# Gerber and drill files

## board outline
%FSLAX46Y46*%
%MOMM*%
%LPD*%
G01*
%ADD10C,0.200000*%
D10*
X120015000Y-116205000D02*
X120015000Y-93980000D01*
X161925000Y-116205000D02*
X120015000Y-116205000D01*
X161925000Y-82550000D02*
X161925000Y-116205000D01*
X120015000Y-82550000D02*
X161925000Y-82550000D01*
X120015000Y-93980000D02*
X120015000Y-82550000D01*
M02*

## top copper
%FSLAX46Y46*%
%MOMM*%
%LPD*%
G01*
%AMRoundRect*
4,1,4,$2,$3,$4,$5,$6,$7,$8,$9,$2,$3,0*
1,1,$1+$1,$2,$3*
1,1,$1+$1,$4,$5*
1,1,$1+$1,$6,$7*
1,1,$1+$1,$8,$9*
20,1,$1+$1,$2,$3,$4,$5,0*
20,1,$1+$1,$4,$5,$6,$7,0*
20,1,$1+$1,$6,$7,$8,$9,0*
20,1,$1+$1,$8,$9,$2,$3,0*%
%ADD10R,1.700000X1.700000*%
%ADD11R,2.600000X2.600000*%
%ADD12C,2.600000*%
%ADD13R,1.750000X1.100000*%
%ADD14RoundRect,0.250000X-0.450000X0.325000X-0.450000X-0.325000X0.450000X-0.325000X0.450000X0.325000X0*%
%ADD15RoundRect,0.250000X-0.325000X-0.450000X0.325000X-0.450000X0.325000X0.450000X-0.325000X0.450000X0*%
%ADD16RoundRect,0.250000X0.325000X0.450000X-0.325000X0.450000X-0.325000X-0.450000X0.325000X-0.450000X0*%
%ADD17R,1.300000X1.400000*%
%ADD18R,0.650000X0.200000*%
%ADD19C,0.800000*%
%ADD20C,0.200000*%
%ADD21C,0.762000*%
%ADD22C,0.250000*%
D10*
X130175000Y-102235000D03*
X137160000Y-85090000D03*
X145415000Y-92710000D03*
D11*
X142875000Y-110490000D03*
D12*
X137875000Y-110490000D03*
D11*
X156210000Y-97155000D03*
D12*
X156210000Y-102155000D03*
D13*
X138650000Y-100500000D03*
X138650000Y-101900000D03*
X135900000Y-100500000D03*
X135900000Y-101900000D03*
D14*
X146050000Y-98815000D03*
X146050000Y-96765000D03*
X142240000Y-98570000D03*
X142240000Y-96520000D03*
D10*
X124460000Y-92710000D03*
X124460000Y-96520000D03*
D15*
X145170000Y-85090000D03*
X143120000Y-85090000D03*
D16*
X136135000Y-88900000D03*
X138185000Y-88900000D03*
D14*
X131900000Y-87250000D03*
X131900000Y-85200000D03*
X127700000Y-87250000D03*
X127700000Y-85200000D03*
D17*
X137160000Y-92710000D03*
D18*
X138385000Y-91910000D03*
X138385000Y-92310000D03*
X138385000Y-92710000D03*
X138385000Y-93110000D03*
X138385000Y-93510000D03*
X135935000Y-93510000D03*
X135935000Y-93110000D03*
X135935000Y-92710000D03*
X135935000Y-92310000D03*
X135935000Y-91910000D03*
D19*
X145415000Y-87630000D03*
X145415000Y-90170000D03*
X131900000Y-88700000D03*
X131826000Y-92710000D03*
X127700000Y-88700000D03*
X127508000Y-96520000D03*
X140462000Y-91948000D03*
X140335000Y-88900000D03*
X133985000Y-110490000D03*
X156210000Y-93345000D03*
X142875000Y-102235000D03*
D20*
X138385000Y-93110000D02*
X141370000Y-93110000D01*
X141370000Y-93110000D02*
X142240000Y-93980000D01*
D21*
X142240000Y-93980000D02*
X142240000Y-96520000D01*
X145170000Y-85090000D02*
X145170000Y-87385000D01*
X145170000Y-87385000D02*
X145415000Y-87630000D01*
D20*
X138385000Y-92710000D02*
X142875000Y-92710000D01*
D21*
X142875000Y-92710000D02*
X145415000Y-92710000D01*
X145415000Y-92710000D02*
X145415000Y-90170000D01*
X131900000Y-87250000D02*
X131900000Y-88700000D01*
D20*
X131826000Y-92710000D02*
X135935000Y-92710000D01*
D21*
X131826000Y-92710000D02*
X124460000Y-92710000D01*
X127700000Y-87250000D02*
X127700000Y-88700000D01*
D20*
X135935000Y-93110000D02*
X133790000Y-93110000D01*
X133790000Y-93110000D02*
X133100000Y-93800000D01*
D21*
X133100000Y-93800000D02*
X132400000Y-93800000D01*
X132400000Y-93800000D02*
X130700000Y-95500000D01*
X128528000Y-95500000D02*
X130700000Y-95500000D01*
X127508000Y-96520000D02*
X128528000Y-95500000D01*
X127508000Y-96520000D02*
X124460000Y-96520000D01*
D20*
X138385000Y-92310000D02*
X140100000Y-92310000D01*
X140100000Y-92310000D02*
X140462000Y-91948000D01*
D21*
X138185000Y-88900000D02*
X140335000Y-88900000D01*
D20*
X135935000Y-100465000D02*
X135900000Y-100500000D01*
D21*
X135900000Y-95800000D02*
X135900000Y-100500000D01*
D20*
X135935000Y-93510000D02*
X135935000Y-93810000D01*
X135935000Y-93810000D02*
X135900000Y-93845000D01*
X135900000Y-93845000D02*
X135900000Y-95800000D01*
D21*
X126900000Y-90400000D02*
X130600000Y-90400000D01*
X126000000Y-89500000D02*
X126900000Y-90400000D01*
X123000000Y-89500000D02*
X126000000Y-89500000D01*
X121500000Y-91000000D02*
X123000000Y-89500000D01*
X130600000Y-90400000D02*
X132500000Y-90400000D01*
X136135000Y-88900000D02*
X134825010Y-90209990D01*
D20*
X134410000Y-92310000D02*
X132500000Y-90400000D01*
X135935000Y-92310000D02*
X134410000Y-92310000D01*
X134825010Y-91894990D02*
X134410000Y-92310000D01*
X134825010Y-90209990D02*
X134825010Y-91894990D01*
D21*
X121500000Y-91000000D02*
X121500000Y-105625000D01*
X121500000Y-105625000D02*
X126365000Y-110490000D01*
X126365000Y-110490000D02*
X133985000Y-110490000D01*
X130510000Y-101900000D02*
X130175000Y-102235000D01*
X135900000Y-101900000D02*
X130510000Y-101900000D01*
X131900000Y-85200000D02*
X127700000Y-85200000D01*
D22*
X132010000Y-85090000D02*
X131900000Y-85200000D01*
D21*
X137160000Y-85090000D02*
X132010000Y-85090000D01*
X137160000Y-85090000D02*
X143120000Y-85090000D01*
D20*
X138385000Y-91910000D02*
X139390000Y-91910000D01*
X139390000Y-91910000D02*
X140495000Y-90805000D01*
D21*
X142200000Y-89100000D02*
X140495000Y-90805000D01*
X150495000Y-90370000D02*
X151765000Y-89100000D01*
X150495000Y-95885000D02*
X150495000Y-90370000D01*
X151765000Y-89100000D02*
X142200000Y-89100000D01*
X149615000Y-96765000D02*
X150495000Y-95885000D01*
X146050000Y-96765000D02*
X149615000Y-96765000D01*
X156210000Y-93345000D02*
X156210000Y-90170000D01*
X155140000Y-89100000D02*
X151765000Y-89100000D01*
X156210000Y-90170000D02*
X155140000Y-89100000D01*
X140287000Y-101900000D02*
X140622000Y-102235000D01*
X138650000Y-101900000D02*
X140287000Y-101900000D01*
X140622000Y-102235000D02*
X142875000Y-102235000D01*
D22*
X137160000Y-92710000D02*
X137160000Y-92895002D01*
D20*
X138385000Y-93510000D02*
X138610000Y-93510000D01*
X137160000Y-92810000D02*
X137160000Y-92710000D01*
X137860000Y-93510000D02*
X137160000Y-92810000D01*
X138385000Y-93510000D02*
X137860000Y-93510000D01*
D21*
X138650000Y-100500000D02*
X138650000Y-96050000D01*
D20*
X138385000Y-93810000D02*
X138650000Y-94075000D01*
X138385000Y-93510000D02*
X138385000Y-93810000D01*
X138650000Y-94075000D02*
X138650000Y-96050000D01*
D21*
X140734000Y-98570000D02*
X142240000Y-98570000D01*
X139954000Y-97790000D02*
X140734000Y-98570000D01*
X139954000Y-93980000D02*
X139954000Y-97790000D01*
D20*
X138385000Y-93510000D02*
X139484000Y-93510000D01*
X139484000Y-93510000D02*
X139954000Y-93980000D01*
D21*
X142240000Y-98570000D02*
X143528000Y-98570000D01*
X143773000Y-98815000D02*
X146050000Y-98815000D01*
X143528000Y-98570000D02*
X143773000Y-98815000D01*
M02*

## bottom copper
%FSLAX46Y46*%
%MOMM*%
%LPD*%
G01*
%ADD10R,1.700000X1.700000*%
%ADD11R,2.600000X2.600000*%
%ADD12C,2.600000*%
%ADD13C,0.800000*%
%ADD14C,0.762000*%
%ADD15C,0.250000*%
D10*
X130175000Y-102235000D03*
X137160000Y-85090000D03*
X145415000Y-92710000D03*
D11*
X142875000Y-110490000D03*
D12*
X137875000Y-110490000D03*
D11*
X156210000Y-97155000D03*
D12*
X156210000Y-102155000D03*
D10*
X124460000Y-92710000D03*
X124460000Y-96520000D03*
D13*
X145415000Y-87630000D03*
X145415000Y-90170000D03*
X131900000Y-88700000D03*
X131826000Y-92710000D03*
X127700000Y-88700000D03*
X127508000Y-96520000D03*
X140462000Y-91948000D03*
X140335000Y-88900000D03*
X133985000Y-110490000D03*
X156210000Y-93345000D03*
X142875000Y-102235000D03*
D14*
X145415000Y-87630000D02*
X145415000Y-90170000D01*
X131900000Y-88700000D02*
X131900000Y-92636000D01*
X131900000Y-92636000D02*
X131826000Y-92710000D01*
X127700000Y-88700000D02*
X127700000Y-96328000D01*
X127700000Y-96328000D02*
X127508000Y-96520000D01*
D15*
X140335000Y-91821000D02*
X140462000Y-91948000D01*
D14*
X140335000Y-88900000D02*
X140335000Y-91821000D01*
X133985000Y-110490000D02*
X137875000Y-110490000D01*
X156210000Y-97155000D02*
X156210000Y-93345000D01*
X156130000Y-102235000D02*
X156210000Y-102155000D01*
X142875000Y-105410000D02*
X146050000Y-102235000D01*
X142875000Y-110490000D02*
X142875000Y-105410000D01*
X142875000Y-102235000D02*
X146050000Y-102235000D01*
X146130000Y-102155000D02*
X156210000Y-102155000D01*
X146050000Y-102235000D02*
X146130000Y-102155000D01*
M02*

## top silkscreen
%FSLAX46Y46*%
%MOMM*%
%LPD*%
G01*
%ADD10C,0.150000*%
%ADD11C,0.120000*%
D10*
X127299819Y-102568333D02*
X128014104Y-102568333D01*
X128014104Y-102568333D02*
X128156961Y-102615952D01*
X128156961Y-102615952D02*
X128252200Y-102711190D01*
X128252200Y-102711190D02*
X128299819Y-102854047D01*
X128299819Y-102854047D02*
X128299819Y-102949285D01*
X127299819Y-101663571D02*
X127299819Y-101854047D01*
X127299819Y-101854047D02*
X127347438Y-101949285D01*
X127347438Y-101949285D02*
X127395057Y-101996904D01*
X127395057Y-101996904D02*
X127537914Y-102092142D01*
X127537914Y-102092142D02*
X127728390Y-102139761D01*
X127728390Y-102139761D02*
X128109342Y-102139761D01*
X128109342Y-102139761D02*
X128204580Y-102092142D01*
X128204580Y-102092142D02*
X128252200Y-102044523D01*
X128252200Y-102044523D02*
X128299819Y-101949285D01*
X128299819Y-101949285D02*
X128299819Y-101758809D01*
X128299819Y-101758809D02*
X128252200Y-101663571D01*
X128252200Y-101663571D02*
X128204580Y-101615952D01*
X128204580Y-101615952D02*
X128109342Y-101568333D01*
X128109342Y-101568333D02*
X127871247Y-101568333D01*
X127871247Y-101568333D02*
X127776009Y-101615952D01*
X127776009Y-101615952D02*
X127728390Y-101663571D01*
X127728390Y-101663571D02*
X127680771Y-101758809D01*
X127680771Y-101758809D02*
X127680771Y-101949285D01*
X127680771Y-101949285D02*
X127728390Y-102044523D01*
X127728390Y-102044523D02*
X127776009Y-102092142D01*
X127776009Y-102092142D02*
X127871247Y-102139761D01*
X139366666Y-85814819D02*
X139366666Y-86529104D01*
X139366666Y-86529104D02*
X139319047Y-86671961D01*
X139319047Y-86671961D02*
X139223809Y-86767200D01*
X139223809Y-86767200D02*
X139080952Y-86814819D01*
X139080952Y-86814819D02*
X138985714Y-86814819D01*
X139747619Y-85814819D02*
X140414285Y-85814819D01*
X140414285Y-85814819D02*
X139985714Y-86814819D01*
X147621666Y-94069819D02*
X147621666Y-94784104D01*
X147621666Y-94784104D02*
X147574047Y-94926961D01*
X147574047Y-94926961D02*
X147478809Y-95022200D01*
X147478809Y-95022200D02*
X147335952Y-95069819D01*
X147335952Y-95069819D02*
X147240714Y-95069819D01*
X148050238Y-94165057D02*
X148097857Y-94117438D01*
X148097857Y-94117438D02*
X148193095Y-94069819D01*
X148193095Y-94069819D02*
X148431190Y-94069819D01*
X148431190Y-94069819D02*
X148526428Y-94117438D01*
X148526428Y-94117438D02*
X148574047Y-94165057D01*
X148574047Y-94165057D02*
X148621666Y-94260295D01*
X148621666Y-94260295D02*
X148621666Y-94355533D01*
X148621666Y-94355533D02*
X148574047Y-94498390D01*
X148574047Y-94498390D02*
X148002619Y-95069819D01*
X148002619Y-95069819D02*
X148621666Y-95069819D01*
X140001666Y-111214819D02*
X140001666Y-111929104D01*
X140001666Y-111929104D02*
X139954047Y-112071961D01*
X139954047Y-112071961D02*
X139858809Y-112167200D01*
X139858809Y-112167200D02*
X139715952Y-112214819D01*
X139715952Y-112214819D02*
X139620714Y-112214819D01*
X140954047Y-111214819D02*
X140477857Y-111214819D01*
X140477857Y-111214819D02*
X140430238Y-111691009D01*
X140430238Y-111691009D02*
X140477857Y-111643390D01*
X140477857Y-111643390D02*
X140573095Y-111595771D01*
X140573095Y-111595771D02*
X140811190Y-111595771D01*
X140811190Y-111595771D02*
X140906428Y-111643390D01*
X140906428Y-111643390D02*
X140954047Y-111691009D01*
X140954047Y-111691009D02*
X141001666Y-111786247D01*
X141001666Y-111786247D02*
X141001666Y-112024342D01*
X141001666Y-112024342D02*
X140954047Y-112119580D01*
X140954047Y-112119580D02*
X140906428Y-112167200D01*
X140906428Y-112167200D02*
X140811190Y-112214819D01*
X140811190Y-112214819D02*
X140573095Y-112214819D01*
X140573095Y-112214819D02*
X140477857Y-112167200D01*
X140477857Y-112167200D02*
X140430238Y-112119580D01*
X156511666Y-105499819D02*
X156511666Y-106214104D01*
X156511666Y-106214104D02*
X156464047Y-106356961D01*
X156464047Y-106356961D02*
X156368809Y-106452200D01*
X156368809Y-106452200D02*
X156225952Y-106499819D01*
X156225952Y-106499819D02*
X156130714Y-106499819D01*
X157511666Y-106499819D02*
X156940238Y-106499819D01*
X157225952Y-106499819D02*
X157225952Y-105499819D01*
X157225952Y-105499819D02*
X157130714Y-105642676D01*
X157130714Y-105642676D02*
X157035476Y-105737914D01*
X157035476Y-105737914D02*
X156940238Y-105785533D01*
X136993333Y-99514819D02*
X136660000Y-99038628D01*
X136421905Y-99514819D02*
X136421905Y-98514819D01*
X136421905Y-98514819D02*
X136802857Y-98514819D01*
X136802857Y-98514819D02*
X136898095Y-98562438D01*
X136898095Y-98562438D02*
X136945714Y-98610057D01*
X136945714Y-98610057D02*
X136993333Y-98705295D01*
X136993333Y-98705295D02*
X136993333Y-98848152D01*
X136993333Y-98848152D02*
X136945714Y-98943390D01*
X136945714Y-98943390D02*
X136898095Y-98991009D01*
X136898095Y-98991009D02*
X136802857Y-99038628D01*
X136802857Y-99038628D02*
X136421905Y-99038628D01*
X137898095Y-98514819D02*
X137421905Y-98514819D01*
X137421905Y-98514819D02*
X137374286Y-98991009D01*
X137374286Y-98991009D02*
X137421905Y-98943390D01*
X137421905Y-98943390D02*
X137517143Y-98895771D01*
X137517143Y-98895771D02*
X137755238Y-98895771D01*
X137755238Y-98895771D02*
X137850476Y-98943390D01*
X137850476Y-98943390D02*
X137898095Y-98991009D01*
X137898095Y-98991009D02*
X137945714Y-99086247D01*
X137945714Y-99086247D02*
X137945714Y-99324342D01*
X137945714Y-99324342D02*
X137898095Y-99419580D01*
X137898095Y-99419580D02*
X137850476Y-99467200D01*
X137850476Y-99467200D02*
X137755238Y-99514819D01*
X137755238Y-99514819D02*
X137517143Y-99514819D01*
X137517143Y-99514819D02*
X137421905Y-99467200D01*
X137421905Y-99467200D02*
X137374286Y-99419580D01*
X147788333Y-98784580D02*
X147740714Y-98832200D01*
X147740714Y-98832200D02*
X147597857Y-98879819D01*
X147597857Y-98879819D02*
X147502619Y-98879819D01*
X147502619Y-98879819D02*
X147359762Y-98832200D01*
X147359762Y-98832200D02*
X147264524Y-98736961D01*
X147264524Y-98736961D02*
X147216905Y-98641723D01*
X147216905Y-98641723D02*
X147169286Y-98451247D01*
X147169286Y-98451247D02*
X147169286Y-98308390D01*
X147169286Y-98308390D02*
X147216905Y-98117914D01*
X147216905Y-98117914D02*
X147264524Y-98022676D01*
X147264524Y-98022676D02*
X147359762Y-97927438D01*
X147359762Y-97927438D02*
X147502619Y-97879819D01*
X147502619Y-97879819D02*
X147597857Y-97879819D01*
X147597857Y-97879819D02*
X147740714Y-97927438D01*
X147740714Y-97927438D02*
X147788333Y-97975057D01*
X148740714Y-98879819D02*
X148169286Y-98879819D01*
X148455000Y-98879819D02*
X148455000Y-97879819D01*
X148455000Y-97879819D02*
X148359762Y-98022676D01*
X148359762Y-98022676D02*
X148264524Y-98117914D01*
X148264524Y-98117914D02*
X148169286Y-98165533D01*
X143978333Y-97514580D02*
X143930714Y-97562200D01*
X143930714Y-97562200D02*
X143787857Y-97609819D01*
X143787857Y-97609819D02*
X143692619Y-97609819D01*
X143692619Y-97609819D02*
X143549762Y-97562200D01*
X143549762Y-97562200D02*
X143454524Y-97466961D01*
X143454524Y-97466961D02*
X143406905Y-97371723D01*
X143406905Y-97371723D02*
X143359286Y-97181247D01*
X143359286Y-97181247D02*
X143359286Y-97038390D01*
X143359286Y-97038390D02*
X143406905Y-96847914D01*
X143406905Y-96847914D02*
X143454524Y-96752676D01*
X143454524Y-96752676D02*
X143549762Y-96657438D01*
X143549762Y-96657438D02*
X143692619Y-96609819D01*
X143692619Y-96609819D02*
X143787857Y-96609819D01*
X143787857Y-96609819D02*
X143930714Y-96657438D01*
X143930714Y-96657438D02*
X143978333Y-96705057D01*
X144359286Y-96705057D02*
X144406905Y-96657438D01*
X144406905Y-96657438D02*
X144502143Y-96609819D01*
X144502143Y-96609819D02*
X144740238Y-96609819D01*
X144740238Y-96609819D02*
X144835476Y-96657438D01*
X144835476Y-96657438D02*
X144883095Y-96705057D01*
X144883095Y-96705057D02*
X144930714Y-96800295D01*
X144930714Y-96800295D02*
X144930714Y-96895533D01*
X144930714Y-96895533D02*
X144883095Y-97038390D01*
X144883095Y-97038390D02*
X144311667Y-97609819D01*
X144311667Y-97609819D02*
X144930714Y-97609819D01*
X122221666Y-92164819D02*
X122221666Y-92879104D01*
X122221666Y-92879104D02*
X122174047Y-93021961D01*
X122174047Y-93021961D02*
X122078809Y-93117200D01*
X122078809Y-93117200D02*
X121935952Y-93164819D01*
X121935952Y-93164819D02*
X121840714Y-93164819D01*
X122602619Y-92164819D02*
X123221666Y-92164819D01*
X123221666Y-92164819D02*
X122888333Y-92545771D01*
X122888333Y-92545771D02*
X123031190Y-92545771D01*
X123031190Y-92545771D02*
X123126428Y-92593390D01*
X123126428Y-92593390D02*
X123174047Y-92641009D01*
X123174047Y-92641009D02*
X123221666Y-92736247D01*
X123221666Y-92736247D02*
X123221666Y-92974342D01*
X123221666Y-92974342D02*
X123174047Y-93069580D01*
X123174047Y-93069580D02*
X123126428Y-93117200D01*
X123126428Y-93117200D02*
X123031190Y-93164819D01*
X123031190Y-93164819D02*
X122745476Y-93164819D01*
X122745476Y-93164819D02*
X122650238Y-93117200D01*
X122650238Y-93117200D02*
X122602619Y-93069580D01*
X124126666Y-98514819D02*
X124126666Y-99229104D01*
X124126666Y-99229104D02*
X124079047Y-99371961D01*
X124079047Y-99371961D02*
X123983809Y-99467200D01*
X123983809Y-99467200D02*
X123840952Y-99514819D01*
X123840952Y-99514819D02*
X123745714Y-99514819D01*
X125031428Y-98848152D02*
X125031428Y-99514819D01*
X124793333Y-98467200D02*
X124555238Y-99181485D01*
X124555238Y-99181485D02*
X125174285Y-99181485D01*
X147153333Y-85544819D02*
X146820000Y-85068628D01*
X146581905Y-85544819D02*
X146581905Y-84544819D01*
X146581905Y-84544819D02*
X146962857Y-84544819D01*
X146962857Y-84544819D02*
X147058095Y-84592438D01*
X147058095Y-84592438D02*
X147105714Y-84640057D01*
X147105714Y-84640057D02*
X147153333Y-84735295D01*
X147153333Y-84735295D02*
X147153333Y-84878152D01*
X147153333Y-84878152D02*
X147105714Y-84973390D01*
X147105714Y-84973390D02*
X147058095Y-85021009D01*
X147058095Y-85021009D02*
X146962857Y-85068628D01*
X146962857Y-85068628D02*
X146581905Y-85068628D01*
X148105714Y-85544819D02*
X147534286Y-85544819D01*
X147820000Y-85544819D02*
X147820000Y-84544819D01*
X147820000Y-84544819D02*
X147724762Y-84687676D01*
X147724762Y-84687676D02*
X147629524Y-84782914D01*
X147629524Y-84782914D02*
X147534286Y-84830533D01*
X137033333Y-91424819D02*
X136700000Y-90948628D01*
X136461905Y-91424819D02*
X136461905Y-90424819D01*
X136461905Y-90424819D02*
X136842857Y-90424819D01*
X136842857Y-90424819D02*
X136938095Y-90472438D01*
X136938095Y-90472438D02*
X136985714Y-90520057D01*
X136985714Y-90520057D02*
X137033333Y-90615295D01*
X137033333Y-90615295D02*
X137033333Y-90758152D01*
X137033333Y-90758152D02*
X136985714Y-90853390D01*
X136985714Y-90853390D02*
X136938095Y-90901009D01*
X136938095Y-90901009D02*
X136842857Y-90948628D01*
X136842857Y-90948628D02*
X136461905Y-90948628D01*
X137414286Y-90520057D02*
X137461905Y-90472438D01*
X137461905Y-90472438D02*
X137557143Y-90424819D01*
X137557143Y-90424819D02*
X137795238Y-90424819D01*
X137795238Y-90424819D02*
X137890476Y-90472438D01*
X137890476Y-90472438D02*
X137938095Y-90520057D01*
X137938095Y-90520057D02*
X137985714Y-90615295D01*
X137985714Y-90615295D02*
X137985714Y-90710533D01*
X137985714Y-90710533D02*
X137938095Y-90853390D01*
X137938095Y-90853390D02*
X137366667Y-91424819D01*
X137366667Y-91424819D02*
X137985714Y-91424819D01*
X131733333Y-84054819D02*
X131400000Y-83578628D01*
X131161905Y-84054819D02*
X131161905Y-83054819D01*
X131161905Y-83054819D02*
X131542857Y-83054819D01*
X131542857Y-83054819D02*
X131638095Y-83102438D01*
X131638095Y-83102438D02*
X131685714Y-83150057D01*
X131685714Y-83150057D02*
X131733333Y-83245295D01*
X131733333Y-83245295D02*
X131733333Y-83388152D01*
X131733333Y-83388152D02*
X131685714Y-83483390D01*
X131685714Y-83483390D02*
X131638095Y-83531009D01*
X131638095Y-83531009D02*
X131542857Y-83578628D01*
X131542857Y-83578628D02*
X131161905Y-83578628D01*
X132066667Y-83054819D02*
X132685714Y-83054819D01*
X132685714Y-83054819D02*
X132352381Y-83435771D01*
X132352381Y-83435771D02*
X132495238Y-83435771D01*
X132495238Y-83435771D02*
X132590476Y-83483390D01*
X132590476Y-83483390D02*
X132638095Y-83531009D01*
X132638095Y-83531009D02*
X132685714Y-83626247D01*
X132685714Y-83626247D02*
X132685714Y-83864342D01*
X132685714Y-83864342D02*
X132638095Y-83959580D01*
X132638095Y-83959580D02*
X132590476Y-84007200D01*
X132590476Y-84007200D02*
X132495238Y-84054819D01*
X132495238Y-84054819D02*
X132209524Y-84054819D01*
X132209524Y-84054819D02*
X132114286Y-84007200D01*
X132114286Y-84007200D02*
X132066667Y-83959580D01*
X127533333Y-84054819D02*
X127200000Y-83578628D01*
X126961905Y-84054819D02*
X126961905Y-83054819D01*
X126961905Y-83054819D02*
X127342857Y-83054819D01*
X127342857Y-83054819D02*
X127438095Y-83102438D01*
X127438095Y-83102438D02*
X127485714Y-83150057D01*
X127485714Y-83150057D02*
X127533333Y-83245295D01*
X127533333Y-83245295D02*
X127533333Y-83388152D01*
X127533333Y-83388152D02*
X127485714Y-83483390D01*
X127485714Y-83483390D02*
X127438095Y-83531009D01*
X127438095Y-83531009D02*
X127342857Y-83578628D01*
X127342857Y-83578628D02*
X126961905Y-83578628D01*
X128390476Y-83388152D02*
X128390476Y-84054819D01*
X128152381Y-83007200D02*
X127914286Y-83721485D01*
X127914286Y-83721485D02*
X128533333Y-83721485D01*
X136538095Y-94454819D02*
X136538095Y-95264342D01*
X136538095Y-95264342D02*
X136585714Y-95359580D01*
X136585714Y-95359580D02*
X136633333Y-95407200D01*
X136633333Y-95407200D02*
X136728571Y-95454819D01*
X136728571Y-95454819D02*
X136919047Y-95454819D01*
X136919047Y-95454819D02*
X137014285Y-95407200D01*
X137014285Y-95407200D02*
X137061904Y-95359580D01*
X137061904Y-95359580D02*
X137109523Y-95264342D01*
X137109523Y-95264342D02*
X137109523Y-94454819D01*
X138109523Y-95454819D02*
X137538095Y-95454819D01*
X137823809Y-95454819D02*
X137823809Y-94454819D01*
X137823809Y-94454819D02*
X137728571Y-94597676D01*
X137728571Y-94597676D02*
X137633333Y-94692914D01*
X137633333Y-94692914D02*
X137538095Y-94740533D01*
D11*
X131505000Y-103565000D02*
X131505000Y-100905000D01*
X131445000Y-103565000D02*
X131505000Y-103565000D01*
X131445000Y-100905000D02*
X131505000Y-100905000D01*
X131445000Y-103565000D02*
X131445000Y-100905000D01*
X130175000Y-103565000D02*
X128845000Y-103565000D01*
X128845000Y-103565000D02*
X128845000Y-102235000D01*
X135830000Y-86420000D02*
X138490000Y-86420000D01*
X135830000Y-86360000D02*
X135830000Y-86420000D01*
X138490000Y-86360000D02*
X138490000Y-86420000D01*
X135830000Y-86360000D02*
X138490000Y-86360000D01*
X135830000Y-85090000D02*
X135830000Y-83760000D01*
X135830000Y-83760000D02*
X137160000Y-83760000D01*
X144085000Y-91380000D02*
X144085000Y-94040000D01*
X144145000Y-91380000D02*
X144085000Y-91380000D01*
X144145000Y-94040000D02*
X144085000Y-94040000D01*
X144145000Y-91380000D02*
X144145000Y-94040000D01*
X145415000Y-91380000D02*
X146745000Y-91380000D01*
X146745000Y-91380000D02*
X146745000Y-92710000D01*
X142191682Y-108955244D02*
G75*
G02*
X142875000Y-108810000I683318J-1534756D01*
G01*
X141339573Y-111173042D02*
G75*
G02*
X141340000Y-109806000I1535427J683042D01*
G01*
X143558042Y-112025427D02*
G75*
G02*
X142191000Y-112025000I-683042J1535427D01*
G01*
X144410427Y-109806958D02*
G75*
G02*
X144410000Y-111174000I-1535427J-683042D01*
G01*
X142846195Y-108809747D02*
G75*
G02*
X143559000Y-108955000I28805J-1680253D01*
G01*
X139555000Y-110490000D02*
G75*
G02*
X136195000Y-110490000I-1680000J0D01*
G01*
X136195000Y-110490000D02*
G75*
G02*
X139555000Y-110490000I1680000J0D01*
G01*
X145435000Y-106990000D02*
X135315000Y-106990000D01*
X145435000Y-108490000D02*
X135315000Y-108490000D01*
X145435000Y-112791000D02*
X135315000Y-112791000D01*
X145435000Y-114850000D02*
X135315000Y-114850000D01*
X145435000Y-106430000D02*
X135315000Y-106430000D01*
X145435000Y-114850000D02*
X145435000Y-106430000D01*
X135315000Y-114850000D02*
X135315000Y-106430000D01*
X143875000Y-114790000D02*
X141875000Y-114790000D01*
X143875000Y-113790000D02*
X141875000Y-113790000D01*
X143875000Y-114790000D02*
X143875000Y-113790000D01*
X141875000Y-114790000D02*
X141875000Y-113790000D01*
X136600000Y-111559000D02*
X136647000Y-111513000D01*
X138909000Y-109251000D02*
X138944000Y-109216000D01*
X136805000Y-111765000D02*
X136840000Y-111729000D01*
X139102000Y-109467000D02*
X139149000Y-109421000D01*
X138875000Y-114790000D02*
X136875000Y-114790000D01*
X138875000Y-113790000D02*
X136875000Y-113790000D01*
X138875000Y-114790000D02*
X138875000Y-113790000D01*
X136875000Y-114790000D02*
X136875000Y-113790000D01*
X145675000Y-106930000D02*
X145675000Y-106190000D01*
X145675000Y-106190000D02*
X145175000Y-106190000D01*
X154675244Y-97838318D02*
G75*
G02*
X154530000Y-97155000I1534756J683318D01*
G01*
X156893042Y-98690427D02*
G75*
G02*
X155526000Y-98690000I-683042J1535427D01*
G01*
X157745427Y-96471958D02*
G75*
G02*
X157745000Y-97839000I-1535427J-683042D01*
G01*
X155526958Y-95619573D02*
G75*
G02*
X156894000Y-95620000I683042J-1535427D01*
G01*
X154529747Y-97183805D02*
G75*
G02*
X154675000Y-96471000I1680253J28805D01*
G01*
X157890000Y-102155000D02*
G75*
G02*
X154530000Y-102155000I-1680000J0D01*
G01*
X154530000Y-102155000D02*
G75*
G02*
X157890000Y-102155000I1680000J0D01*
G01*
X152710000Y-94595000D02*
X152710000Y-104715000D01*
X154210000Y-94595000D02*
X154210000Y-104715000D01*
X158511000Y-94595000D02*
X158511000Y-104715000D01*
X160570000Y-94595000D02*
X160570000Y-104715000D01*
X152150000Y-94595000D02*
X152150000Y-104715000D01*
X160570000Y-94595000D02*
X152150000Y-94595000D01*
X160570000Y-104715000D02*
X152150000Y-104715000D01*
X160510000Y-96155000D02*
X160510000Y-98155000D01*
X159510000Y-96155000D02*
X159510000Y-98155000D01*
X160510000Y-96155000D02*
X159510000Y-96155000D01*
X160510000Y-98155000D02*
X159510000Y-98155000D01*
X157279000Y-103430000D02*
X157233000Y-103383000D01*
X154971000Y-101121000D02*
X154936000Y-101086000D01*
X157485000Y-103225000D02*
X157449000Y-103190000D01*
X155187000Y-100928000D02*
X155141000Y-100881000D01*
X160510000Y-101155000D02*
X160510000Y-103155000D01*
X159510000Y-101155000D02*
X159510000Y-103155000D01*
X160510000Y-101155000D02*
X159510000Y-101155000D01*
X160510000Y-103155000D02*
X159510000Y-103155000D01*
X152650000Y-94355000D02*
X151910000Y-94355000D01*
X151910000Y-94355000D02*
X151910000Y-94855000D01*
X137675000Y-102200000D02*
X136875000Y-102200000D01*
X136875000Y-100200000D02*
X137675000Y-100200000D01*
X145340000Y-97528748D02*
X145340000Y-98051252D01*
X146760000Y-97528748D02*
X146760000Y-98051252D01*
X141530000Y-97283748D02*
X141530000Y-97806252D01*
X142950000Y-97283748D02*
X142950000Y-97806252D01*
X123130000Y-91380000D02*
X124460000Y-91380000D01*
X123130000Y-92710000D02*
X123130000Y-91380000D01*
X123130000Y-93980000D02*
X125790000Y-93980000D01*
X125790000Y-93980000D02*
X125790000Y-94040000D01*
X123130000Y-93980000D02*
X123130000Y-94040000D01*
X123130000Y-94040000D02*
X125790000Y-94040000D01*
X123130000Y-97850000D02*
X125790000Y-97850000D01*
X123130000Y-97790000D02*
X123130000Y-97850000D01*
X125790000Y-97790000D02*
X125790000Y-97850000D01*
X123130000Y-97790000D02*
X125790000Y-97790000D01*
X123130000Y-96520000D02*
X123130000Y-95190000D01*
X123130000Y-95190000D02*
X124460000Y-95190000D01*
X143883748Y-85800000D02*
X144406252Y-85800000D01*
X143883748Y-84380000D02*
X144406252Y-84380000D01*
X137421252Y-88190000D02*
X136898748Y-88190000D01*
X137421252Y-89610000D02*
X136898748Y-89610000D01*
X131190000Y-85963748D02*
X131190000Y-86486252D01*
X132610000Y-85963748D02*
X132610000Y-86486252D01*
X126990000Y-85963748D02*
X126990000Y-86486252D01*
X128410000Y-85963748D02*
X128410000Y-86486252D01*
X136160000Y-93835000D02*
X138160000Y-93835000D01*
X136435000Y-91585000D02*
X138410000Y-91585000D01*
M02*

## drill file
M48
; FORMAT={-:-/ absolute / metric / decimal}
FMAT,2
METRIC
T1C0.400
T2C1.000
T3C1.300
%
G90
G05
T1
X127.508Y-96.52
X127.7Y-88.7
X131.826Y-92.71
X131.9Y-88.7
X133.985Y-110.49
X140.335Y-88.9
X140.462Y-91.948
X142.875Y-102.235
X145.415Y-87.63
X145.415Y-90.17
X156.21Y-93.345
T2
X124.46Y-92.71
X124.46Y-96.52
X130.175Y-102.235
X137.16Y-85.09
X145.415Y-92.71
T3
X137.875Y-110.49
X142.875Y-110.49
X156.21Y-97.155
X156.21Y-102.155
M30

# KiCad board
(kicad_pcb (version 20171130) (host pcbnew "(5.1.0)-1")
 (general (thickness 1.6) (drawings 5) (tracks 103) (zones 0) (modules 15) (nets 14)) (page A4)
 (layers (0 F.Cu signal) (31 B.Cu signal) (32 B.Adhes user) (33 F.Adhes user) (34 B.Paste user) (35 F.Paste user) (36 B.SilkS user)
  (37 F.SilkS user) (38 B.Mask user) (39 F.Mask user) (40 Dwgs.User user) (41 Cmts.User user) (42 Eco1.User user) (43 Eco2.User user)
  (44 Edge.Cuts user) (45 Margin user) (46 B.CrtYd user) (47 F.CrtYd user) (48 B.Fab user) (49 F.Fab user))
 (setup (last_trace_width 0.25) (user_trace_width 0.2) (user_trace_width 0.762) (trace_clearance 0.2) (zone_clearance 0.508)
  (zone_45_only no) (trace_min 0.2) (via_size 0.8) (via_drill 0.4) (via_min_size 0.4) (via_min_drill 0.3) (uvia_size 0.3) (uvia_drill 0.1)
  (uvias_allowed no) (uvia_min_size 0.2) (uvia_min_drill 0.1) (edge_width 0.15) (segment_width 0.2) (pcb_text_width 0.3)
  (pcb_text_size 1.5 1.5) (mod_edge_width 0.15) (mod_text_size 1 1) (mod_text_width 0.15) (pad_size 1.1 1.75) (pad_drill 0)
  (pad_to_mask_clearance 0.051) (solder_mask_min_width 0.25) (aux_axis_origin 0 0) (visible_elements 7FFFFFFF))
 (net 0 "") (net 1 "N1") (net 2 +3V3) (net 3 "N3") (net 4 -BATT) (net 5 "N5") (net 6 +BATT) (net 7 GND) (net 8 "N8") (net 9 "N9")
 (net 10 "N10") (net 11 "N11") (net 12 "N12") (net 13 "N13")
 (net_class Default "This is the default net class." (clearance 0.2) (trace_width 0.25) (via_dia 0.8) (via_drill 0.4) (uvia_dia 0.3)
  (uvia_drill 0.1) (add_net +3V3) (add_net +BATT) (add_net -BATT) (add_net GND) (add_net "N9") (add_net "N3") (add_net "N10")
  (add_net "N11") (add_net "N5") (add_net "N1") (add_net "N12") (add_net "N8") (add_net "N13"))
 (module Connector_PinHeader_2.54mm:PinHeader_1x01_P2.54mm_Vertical (layer F.Cu) (at 130.175 102.235 90)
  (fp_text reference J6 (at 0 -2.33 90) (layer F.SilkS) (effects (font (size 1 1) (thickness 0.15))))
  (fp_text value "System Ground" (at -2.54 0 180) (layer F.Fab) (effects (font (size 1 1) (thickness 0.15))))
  (fp_line (start -1.33 1.33) (end 1.33 1.33) (layer F.SilkS) (width 0.12))
  (fp_line (start -1.33 1.27) (end -1.33 1.33) (layer F.SilkS) (width 0.12))
  (fp_line (start 1.33 1.27) (end 1.33 1.33) (layer F.SilkS) (width 0.12))
  (fp_line (start -1.33 1.27) (end 1.33 1.27) (layer F.SilkS) (width 0.12))
  (fp_line (start -1.33 0) (end -1.33 -1.33) (layer F.SilkS) (width 0.12))
  (fp_line (start -1.33 -1.33) (end 0 -1.33) (layer F.SilkS) (width 0.12))
  (pad 1 thru_hole rect (at 0 0 90) (size 1.7 1.7) (drill 1) (layers *.Cu *.Mask) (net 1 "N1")))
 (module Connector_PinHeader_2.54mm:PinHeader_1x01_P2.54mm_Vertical (layer F.Cu) (at 137.16 85.09)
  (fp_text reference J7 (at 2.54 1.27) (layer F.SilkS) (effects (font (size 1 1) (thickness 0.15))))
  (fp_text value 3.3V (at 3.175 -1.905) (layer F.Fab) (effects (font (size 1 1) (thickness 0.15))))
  (fp_line (start -1.33 1.33) (end 1.33 1.33) (layer F.SilkS) (width 0.12))
  (fp_line (start -1.33 1.27) (end -1.33 1.33) (layer F.SilkS) (width 0.12))
  (fp_line (start 1.33 1.27) (end 1.33 1.33) (layer F.SilkS) (width 0.12))
  (fp_line (start -1.33 1.27) (end 1.33 1.27) (layer F.SilkS) (width 0.12))
  (fp_line (start -1.33 0) (end -1.33 -1.33) (layer F.SilkS) (width 0.12))
  (fp_line (start -1.33 -1.33) (end 0 -1.33) (layer F.SilkS) (width 0.12))
  (pad 1 thru_hole rect (at 0 0) (size 1.7 1.7) (drill 1) (layers *.Cu *.Mask) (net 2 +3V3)))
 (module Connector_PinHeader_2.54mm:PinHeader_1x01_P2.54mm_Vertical (layer F.Cu) (at 145.415 92.71 270)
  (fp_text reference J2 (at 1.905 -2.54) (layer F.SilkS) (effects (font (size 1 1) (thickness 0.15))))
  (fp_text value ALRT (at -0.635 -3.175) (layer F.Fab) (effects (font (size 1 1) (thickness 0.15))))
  (fp_line (start -1.33 1.33) (end 1.33 1.33) (layer F.SilkS) (width 0.12))
  (fp_line (start -1.33 1.27) (end -1.33 1.33) (layer F.SilkS) (width 0.12))
  (fp_line (start 1.33 1.27) (end 1.33 1.33) (layer F.SilkS) (width 0.12))
  (fp_line (start -1.33 1.27) (end 1.33 1.27) (layer F.SilkS) (width 0.12))
  (fp_line (start -1.33 0) (end -1.33 -1.33) (layer F.SilkS) (width 0.12))
  (fp_line (start -1.33 -1.33) (end 0 -1.33) (layer F.SilkS) (width 0.12))
  (pad 1 thru_hole rect (at 0 0 270) (size 1.7 1.7) (drill 1) (layers *.Cu *.Mask) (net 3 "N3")))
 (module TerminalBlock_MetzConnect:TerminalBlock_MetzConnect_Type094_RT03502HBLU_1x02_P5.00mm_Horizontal (layer F.Cu)
  (at 142.875 110.49 180)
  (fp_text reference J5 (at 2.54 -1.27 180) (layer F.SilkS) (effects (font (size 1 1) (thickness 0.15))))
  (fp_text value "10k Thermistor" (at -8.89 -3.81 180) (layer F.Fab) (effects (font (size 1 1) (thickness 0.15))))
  (fp_arc (start 0 0) (end 0 1.68) (angle -24) (layer F.SilkS) (width 0.12))
  (fp_arc (start 0 0) (end 1.535 0.684) (angle -48) (layer F.SilkS) (width 0.12))
  (fp_arc (start 0 0) (end 0.684 -1.535) (angle -48) (layer F.SilkS) (width 0.12))
  (fp_arc (start 0 0) (end -1.535 -0.684) (angle -48) (layer F.SilkS) (width 0.12))
  (fp_arc (start 0 0) (end -0.684 1.535) (angle -25) (layer F.SilkS) (width 0.12))
  (fp_circle (center 5 0) (end 6.68 0) (layer F.SilkS) (width 0.12))
  (fp_line (start -2.56 3.5) (end 7.56 3.5) (layer F.SilkS) (width 0.12))
  (fp_line (start -2.56 2) (end 7.56 2) (layer F.SilkS) (width 0.12))
  (fp_line (start -2.56 -2.301) (end 7.56 -2.301) (layer F.SilkS) (width 0.12))
  (fp_line (start -2.56 -4.36) (end 7.56 -4.36) (layer F.SilkS) (width 0.12))
  (fp_line (start -2.56 4.06) (end 7.56 4.06) (layer F.SilkS) (width 0.12))
  (fp_line (start -2.56 -4.36) (end -2.56 4.06) (layer F.SilkS) (width 0.12))
  (fp_line (start 7.56 -4.36) (end 7.56 4.06) (layer F.SilkS) (width 0.12))
  (fp_line (start -1 -4.3) (end 1 -4.3) (layer F.SilkS) (width 0.12))
  (fp_line (start -1 -3.3) (end 1 -3.3) (layer F.SilkS) (width 0.12))
  (fp_line (start -1 -4.3) (end -1 -3.3) (layer F.SilkS) (width 0.12))
  (fp_line (start 1 -4.3) (end 1 -3.3) (layer F.SilkS) (width 0.12))
  (fp_line (start 6.275 -1.069) (end 6.228 -1.023) (layer F.SilkS) (width 0.12))
  (fp_line (start 3.966 1.239) (end 3.931 1.274) (layer F.SilkS) (width 0.12))
  (fp_line (start 6.07 -1.275) (end 6.035 -1.239) (layer F.SilkS) (width 0.12))
  (fp_line (start 3.773 1.023) (end 3.726 1.069) (layer F.SilkS) (width 0.12))
  (fp_line (start 4 -4.3) (end 6 -4.3) (layer F.SilkS) (width 0.12))
  (fp_line (start 4 -3.3) (end 6 -3.3) (layer F.SilkS) (width 0.12))
  (fp_line (start 4 -4.3) (end 4 -3.3) (layer F.SilkS) (width 0.12))
  (fp_line (start 6 -4.3) (end 6 -3.3) (layer F.SilkS) (width 0.12))
  (fp_line (start -2.8 3.56) (end -2.8 4.3) (layer F.SilkS) (width 0.12))
  (fp_line (start -2.8 4.3) (end -2.3 4.3) (layer F.SilkS) (width 0.12))
  (pad 1 thru_hole rect (at 0 0 180) (size 2.6 2.6) (drill 1.3) (layers *.Cu *.Mask) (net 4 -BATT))
  (pad 2 thru_hole circle (at 5 0 180) (size 2.6 2.6) (drill 1.3) (layers *.Cu *.Mask) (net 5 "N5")))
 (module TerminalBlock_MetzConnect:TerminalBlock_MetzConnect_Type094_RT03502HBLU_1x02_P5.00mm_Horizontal (layer F.Cu) (at 156.21 97.155 270)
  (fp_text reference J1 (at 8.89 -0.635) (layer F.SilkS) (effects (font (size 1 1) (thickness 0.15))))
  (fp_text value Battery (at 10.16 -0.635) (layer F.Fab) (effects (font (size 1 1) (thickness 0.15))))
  (fp_arc (start 0 0) (end 0 1.68) (angle -24) (layer F.SilkS) (width 0.12))
  (fp_arc (start 0 0) (end 1.535 0.684) (angle -48) (layer F.SilkS) (width 0.12))
  (fp_arc (start 0 0) (end 0.684 -1.535) (angle -48) (layer F.SilkS) (width 0.12))
  (fp_arc (start 0 0) (end -1.535 -0.684) (angle -48) (layer F.SilkS) (width 0.12))
  (fp_arc (start 0 0) (end -0.684 1.535) (angle -25) (layer F.SilkS) (width 0.12))
  (fp_circle (center 5 0) (end 6.68 0) (layer F.SilkS) (width 0.12))
  (fp_line (start -2.56 3.5) (end 7.56 3.5) (layer F.SilkS) (width 0.12))
  (fp_line (start -2.56 2) (end 7.56 2) (layer F.SilkS) (width 0.12))
  (fp_line (start -2.56 -2.301) (end 7.56 -2.301) (layer F.SilkS) (width 0.12))
  (fp_line (start -2.56 -4.36) (end 7.56 -4.36) (layer F.SilkS) (width 0.12))
  (fp_line (start -2.56 4.06) (end 7.56 4.06) (layer F.SilkS) (width 0.12))
  (fp_line (start -2.56 -4.36) (end -2.56 4.06) (layer F.SilkS) (width 0.12))
  (fp_line (start 7.56 -4.36) (end 7.56 4.06) (layer F.SilkS) (width 0.12))
  (fp_line (start -1 -4.3) (end 1 -4.3) (layer F.SilkS) (width 0.12))
  (fp_line (start -1 -3.3) (end 1 -3.3) (layer F.SilkS) (width 0.12))
  (fp_line (start -1 -4.3) (end -1 -3.3) (layer F.SilkS) (width 0.12))
  (fp_line (start 1 -4.3) (end 1 -3.3) (layer F.SilkS) (width 0.12))
  (fp_line (start 6.275 -1.069) (end 6.228 -1.023) (layer F.SilkS) (width 0.12))
  (fp_line (start 3.966 1.239) (end 3.931 1.274) (layer F.SilkS) (width 0.12))
  (fp_line (start 6.07 -1.275) (end 6.035 -1.239) (layer F.SilkS) (width 0.12))
  (fp_line (start 3.773 1.023) (end 3.726 1.069) (layer F.SilkS) (width 0.12))
  (fp_line (start 4 -4.3) (end 6 -4.3) (layer F.SilkS) (width 0.12))
  (fp_line (start 4 -3.3) (end 6 -3.3) (layer F.SilkS) (width 0.12))
  (fp_line (start 4 -4.3) (end 4 -3.3) (layer F.SilkS) (width 0.12))
  (fp_line (start 6 -4.3) (end 6 -3.3) (layer F.SilkS) (width 0.12))
  (fp_line (start -2.8 3.56) (end -2.8 4.3) (layer F.SilkS) (width 0.12))
  (fp_line (start -2.8 4.3) (end -2.3 4.3) (layer F.SilkS) (width 0.12))
  (pad 1 thru_hole rect (at 0 0 270) (size 2.6 2.6) (drill 1.3) (layers *.Cu *.Mask) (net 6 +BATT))
  (pad 2 thru_hole circle (at 5 0 270) (size 2.6 2.6) (drill 1.3) (layers *.Cu *.Mask) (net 4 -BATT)))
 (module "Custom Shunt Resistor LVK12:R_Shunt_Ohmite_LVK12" (layer F.Cu) (at 137.275 101.2 90)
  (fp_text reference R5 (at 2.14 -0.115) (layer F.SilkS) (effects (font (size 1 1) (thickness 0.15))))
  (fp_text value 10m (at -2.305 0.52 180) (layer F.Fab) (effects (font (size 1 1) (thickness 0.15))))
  (fp_line (start -1 0.4) (end -1 -0.4) (layer F.SilkS) (width 0.12))
  (fp_line (start 1 -0.4) (end 1 0.4) (layer F.SilkS) (width 0.12))
  (pad 3 smd rect (at 0.7 1.375 90) (size 1.1 1.75) (layers F.Cu F.Paste F.Mask) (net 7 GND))
  (pad 4 smd rect (at -0.7 1.375 90) (size 1.1 1.75) (layers F.Cu F.Paste F.Mask) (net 4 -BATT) (die_length 2))
  (pad 2 smd rect (at 0.7 -1.375 90) (size 1.1 1.75) (layers F.Cu F.Paste F.Mask) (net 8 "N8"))
  (pad 1 smd rect (at -0.7 -1.375 90) (size 1.1 1.75) (layers F.Cu F.Paste F.Mask) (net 1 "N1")))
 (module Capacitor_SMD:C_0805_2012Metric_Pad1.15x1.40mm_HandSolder (layer F.Cu) (at 146.05 97.79 270)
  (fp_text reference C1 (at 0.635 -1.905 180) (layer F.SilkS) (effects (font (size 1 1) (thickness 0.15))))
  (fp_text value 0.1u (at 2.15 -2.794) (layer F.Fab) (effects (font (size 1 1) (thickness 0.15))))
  (fp_line (start -0.261252 0.71) (end 0.261252 0.71) (layer F.SilkS) (width 0.12))
  (fp_line (start -0.261252 -0.71) (end 0.261252 -0.71) (layer F.SilkS) (width 0.12))
  (pad 2 smd roundrect (at 1.025 0 270) (size 1.15 1.4) (layers F.Cu F.Paste F.Mask) (roundrect_rratio 0.217391) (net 7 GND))
  (pad 1 smd roundrect (at -1.025 0 270) (size 1.15 1.4) (layers F.Cu F.Paste F.Mask) (roundrect_rratio 0.217391) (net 6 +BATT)))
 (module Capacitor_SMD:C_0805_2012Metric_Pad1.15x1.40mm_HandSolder (layer F.Cu) (at 142.24 97.545 270)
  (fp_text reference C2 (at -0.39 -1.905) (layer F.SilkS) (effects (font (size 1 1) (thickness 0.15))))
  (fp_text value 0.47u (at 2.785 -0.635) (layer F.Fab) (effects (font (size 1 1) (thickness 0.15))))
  (fp_line (start -0.261252 0.71) (end 0.261252 0.71) (layer F.SilkS) (width 0.12))
  (fp_line (start -0.261252 -0.71) (end 0.261252 -0.71) (layer F.SilkS) (width 0.12))
  (pad 2 smd roundrect (at 1.025 0 270) (size 1.15 1.4) (layers F.Cu F.Paste F.Mask) (roundrect_rratio 0.217391) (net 7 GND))
  (pad 1 smd roundrect (at -1.025 0 270) (size 1.15 1.4) (layers F.Cu F.Paste F.Mask) (roundrect_rratio 0.217391) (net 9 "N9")))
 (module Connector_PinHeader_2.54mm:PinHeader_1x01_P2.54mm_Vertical (layer F.Cu) (at 124.46 92.71)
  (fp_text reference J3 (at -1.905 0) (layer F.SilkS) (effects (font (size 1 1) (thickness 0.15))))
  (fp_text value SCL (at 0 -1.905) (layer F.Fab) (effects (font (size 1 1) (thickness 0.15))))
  (fp_line (start -1.33 -1.33) (end 0 -1.33) (layer F.SilkS) (width 0.12))
  (fp_line (start -1.33 0) (end -1.33 -1.33) (layer F.SilkS) (width 0.12))
  (fp_line (start -1.33 1.27) (end 1.33 1.27) (layer F.SilkS) (width 0.12))
  (fp_line (start 1.33 1.27) (end 1.33 1.33) (layer F.SilkS) (width 0.12))
  (fp_line (start -1.33 1.27) (end -1.33 1.33) (layer F.SilkS) (width 0.12))
  (fp_line (start -1.33 1.33) (end 1.33 1.33) (layer F.SilkS) (width 0.12))
  (pad 1 thru_hole rect (at 0 0) (size 1.7 1.7) (drill 1) (layers *.Cu *.Mask) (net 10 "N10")))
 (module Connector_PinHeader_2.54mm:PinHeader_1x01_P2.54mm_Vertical (layer F.Cu) (at 124.46 96.52)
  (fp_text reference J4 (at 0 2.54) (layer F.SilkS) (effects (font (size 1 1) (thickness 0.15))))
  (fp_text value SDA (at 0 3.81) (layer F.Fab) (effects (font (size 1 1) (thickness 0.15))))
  (fp_line (start -1.33 1.33) (end 1.33 1.33) (layer F.SilkS) (width 0.12))
  (fp_line (start -1.33 1.27) (end -1.33 1.33) (layer F.SilkS) (width 0.12))
  (fp_line (start 1.33 1.27) (end 1.33 1.33) (layer F.SilkS) (width 0.12))
  (fp_line (start -1.33 1.27) (end 1.33 1.27) (layer F.SilkS) (width 0.12))
  (fp_line (start -1.33 0) (end -1.33 -1.33) (layer F.SilkS) (width 0.12))
  (fp_line (start -1.33 -1.33) (end 0 -1.33) (layer F.SilkS) (width 0.12))
  (pad 1 thru_hole rect (at 0 0) (size 1.7 1.7) (drill 1) (layers *.Cu *.Mask) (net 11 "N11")))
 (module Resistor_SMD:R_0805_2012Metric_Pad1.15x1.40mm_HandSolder (layer F.Cu) (at 144.145 85.09)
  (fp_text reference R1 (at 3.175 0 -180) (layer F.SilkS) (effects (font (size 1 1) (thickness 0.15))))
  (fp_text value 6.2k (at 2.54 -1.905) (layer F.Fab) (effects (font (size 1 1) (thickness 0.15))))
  (fp_line (start -0.261252 0.71) (end 0.261252 0.71) (layer F.SilkS) (width 0.12))
  (fp_line (start -0.261252 -0.71) (end 0.261252 -0.71) (layer F.SilkS) (width 0.12))
  (pad 2 smd roundrect (at 1.025 0) (size 1.15 1.4) (layers F.Cu F.Paste F.Mask) (roundrect_rratio 0.217391) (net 3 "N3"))
  (pad 1 smd roundrect (at -1.025 0) (size 1.15 1.4) (layers F.Cu F.Paste F.Mask) (roundrect_rratio 0.217391) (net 2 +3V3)))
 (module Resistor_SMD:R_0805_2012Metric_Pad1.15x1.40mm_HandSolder (layer F.Cu) (at 137.16 88.9 180)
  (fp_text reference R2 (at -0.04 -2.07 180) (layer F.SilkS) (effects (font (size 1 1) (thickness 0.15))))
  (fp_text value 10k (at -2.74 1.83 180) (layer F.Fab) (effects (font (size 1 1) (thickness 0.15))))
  (fp_line (start -0.261252 0.71) (end 0.261252 0.71) (layer F.SilkS) (width 0.12))
  (fp_line (start -0.261252 -0.71) (end 0.261252 -0.71) (layer F.SilkS) (width 0.12))
  (pad 2 smd roundrect (at 1.025 0 180) (size 1.15 1.4) (layers F.Cu F.Paste F.Mask) (roundrect_rratio 0.217391) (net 5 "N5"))
  (pad 1 smd roundrect (at -1.025 0 180) (size 1.15 1.4) (layers F.Cu F.Paste F.Mask) (roundrect_rratio 0.217391) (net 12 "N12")))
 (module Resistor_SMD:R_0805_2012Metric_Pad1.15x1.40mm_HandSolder (layer F.Cu) (at 131.9 86.225 270)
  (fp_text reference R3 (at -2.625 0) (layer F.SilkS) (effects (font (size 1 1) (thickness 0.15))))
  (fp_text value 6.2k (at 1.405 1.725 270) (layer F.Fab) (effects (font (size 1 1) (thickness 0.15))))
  (fp_line (start -0.261252 0.71) (end 0.261252 0.71) (layer F.SilkS) (width 0.12))
  (fp_line (start -0.261252 -0.71) (end 0.261252 -0.71) (layer F.SilkS) (width 0.12))
  (pad 2 smd roundrect (at 1.025 0 270) (size 1.15 1.4) (layers F.Cu F.Paste F.Mask) (roundrect_rratio 0.217391) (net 10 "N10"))
  (pad 1 smd roundrect (at -1.025 0 270) (size 1.15 1.4) (layers F.Cu F.Paste F.Mask) (roundrect_rratio 0.217391) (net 2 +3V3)))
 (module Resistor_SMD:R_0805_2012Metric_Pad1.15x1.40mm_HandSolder (layer F.Cu) (at 127.7 86.225 270)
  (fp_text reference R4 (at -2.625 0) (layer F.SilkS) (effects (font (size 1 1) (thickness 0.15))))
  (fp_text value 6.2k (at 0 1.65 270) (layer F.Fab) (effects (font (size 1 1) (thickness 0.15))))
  (fp_line (start -0.261252 0.71) (end 0.261252 0.71) (layer F.SilkS) (width 0.12))
  (fp_line (start -0.261252 -0.71) (end 0.261252 -0.71) (layer F.SilkS) (width 0.12))
  (pad 2 smd roundrect (at 1.025 0 270) (size 1.15 1.4) (layers F.Cu F.Paste F.Mask) (roundrect_rratio 0.217391) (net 11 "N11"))
  (pad 1 smd roundrect (at -1.025 0 270) (size 1.15 1.4) (layers F.Cu F.Paste F.Mask) (roundrect_rratio 0.217391) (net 2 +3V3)))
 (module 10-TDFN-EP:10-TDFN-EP (layer F.Cu) (at 137.16 92.71)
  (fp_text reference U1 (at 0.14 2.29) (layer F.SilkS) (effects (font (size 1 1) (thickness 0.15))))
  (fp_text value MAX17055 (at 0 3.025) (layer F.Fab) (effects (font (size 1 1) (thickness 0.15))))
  (fp_line (start -1 1.125) (end 1 1.125) (layer F.SilkS) (width 0.12))
  (fp_line (start -0.725 -1.125) (end 1.25 -1.125) (layer F.SilkS) (width 0.12))
  (pad 11 smd rect (at 0 0) (size 1.3 1.4) (layers F.Cu F.Mask) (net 7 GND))
  (pad 10 smd rect (at 1.225 -0.8) (size 0.65 0.2) (layers F.Cu F.Paste F.Mask) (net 6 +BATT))
  (pad 9 smd rect (at 1.225 -0.4) (size 0.65 0.2) (layers F.Cu F.Paste F.Mask) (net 12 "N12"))
  (pad 8 smd rect (at 1.225 0) (size 0.65 0.2) (layers F.Cu F.Paste F.Mask) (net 3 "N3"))
  (pad 7 smd rect (at 1.225 0.4) (size 0.65 0.2) (layers F.Cu F.Paste F.Mask) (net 9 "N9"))
  (pad 6 smd rect (at 1.225 0.8) (size 0.65 0.2) (layers F.Cu F.Paste F.Mask) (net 7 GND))
  (pad 5 smd rect (at -1.225 0.8) (size 0.65 0.2) (layers F.Cu F.Paste F.Mask) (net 8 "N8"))
  (pad 4 smd rect (at -1.225 0.4) (size 0.65 0.2) (layers F.Cu F.Paste F.Mask) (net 11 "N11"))
  (pad 3 smd rect (at -1.225 0) (size 0.65 0.2) (layers F.Cu F.Paste F.Mask) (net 10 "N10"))
  (pad 2 smd rect (at -1.225 -0.4) (size 0.65 0.2) (layers F.Cu F.Paste F.Mask) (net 5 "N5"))
  (pad 1 smd rect (at -1.225 -0.8) (size 0.65 0.2) (layers F.Cu F.Paste F.Mask) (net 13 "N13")))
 (gr_line (start 120.015 116.205) (end 120.015 93.98) (layer Edge.Cuts) (width 0.2))
 (gr_line (start 161.925 116.205) (end 120.015 116.205) (layer Edge.Cuts) (width 0.2))
 (gr_line (start 161.925 82.55) (end 161.925 116.205) (layer Edge.Cuts) (width 0.2))
 (gr_line (start 120.015 82.55) (end 161.925 82.55) (layer Edge.Cuts) (width 0.2))
 (gr_line (start 120.015 93.98) (end 120.015 82.55) (layer Edge.Cuts) (width 0.2))
 (segment (start 138.385 93.11) (end 141.37 93.11) (width 0.2) (layer F.Cu) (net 9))
 (segment (start 141.37 93.11) (end 142.24 93.98) (width 0.2) (layer F.Cu) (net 9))
 (segment (start 142.24 93.98) (end 142.24 96.52) (width 0.762) (layer F.Cu) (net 9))
 (via (at 145.415 87.63) (size 0.8) (drill 0.4) (layers F.Cu B.Cu) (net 3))
 (segment (start 145.17 85.09) (end 145.17 87.385) (width 0.762) (layer F.Cu) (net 3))
 (segment (start 145.17 87.385) (end 145.415 87.63) (width 0.762) (layer F.Cu) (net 3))
 (via (at 145.415 90.17) (size 0.8) (drill 0.4) (layers F.Cu B.Cu) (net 3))
 (segment (start 145.415 87.63) (end 145.415 90.17) (width 0.762) (layer B.Cu) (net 3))
 (segment (start 138.385 92.71) (end 142.875 92.71) (width 0.2) (layer F.Cu) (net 3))
 (segment (start 142.875 92.71) (end 145.415 92.71) (width 0.762) (layer F.Cu) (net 3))
 (segment (start 145.415 92.71) (end 145.415 90.17) (width 0.762) (layer F.Cu) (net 3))
 (via (at 131.9 88.7) (size 0.8) (drill 0.4) (layers F.Cu B.Cu) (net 10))
 (segment (start 131.9 87.25) (end 131.9 88.7) (width 0.762) (layer F.Cu) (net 10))
 (via (at 131.826 92.71) (size 0.8) (drill 0.4) (layers F.Cu B.Cu) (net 10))
 (segment (start 131.9 88.7) (end 131.9 92.636) (width 0.762) (layer B.Cu) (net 10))
 (segment (start 131.9 92.636) (end 131.826 92.71) (width 0.762) (layer B.Cu) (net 10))
 (segment (start 131.826 92.71) (end 135.935 92.71) (width 0.2) (layer F.Cu) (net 10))
 (segment (start 131.826 92.71) (end 124.46 92.71) (width 0.762) (layer F.Cu) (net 10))
 (via (at 127.7 88.7) (size 0.8) (drill 0.4) (layers F.Cu B.Cu) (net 11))
 (segment (start 127.7 87.25) (end 127.7 88.7) (width 0.762) (layer F.Cu) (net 11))
 (segment (start 135.935 93.11) (end 133.79 93.11) (width 0.2) (layer F.Cu) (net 11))
 (segment (start 133.79 93.11) (end 133.1 93.8) (width 0.2) (layer F.Cu) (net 11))
 (segment (start 133.1 93.8) (end 132.4 93.8) (width 0.762) (layer F.Cu) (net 11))
 (segment (start 132.4 93.8) (end 130.7 95.5) (width 0.762) (layer F.Cu) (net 11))
 (via (at 127.508 96.52) (size 0.8) (drill 0.4) (layers F.Cu B.Cu) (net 11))
 (segment (start 127.7 88.7) (end 127.7 96.328) (width 0.762) (layer B.Cu) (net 11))
 (segment (start 127.7 96.328) (end 127.508 96.52) (width 0.762) (layer B.Cu) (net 11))
 (segment (start 128.528 95.5) (end 130.7 95.5) (width 0.762) (layer F.Cu) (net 11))
 (segment (start 127.508 96.52) (end 128.528 95.5) (width 0.762) (layer F.Cu) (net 11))
 (segment (start 127.508 96.52) (end 124.46 96.52) (width 0.762) (layer F.Cu) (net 11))
 (segment (start 138.385 92.31) (end 140.1 92.31) (width 0.2) (layer F.Cu) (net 12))
 (segment (start 140.1 92.31) (end 140.462 91.948) (width 0.2) (layer F.Cu) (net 12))
 (via (at 140.462 91.948) (size 0.8) (drill 0.4) (layers F.Cu B.Cu) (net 12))
 (via (at 140.335 88.9) (size 0.8) (drill 0.4) (layers F.Cu B.Cu) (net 12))
 (segment (start 138.185 88.9) (end 140.335 88.9) (width 0.762) (layer F.Cu) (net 12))
 (segment (start 140.335 91.821) (end 140.462 91.948) (width 0.25) (layer B.Cu) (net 12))
 (segment (start 140.335 88.9) (end 140.335 91.821) (width 0.762) (layer B.Cu) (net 12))
 (segment (start 135.935 100.465) (end 135.9 100.5) (width 0.2) (layer F.Cu) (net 8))
 (segment (start 135.9 95.8) (end 135.9 100.5) (width 0.762) (layer F.Cu) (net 8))
 (segment (start 135.935 93.51) (end 135.935 93.81) (width 0.2) (layer F.Cu) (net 8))
 (segment (start 135.935 93.81) (end 135.9 93.845) (width 0.2) (layer F.Cu) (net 8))
 (segment (start 135.9 93.845) (end 135.9 95.8) (width 0.2) (layer F.Cu) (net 8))
 (segment (start 126.9 90.4) (end 130.6 90.4) (width 0.762) (layer F.Cu) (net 5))
 (segment (start 126 89.5) (end 126.9 90.4) (width 0.762) (layer F.Cu) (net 5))
 (segment (start 123 89.5) (end 126 89.5) (width 0.762) (layer F.Cu) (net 5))
 (segment (start 121.5 91) (end 123 89.5) (width 0.762) (layer F.Cu) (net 5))
 (segment (start 130.6 90.4) (end 132.5 90.4) (width 0.762) (layer F.Cu) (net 5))
 (segment (start 136.135 88.9) (end 134.82501 90.20999) (width 0.762) (layer F.Cu) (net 5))
 (segment (start 134.41 92.31) (end 132.5 90.4) (width 0.2) (layer F.Cu) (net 5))
 (segment (start 135.935 92.31) (end 134.41 92.31) (width 0.2) (layer F.Cu) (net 5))
 (segment (start 134.82501 91.89499) (end 134.41 92.31) (width 0.2) (layer F.Cu) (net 5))
 (segment (start 134.82501 90.20999) (end 134.82501 91.89499) (width 0.2) (layer F.Cu) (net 5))
 (segment (start 121.5 91) (end 121.5 105.625) (width 0.762) (layer F.Cu) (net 5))
 (segment (start 121.5 105.625) (end 126.365 110.49) (width 0.762) (layer F.Cu) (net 5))
 (via (at 133.985 110.49) (size 0.8) (drill 0.4) (layers F.Cu B.Cu) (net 5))
 (segment (start 126.365 110.49) (end 133.985 110.49) (width 0.762) (layer F.Cu) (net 5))
 (segment (start 133.985 110.49) (end 137.875 110.49) (width 0.762) (layer B.Cu) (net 5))
 (segment (start 130.51 101.9) (end 130.175 102.235) (width 0.762) (layer F.Cu) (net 1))
 (segment (start 135.9 101.9) (end 130.51 101.9) (width 0.762) (layer F.Cu) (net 1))
 (segment (start 131.9 85.2) (end 127.7 85.2) (width 0.762) (layer F.Cu) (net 2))
 (segment (start 132.01 85.09) (end 131.9 85.2) (width 0.25) (layer F.Cu) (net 2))
 (segment (start 137.16 85.09) (end 132.01 85.09) (width 0.762) (layer F.Cu) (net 2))
 (segment (start 137.16 85.09) (end 143.12 85.09) (width 0.762) (layer F.Cu) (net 2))
 (segment (start 138.385 91.91) (end 139.39 91.91) (width 0.2) (layer F.Cu) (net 6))
 (segment (start 139.39 91.91) (end 140.495 90.805) (width 0.2) (layer F.Cu) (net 6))
 (segment (start 142.2 89.1) (end 140.495 90.805) (width 0.762) (layer F.Cu) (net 6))
 (segment (start 150.495 90.37) (end 151.765 89.1) (width 0.762) (layer F.Cu) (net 6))
 (segment (start 150.495 95.885) (end 150.495 90.37) (width 0.762) (layer F.Cu) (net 6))
 (segment (start 151.765 89.1) (end 142.2 89.1) (width 0.762) (layer F.Cu) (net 6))
 (segment (start 149.615 96.765) (end 150.495 95.885) (width 0.762) (layer F.Cu) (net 6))
 (segment (start 146.05 96.765) (end 149.615 96.765) (width 0.762) (layer F.Cu) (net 6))
 (via (at 156.21 93.345) (size 0.8) (drill 0.4) (layers F.Cu B.Cu) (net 6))
 (segment (start 156.21 97.155) (end 156.21 93.345) (width 0.762) (layer B.Cu) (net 6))
 (segment (start 156.21 93.345) (end 156.21 90.17) (width 0.762) (layer F.Cu) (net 6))
 (segment (start 155.14 89.1) (end 151.765 89.1) (width 0.762) (layer F.Cu) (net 6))
 (segment (start 156.21 90.17) (end 155.14 89.1) (width 0.762) (layer F.Cu) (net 6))
 (segment (start 140.287 101.9) (end 140.622 102.235) (width 0.762) (layer F.Cu) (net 4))
 (segment (start 138.65 101.9) (end 140.287 101.9) (width 0.762) (layer F.Cu) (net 4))
 (via (at 142.875 102.235) (size 0.8) (drill 0.4) (layers F.Cu B.Cu) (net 4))
 (segment (start 156.13 102.235) (end 156.21 102.155) (width 0.762) (layer B.Cu) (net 4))
 (segment (start 140.622 102.235) (end 142.875 102.235) (width 0.762) (layer F.Cu) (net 4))
 (segment (start 142.875 105.41) (end 146.05 102.235) (width 0.762) (layer B.Cu) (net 4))
 (segment (start 142.875 110.49) (end 142.875 105.41) (width 0.762) (layer B.Cu) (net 4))
 (segment (start 142.875 102.235) (end 146.05 102.235) (width 0.762) (layer B.Cu) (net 4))
 (segment (start 146.13 102.155) (end 156.21 102.155) (width 0.762) (layer B.Cu) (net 4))
 (segment (start 146.05 102.235) (end 146.13 102.155) (width 0.762) (layer B.Cu) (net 4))
 (segment (start 137.16 92.71) (end 137.16 92.895002) (width 0.25) (layer F.Cu) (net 7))
 (segment (start 138.385 93.51) (end 138.61 93.51) (width 0.2) (layer F.Cu) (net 7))
 (segment (start 137.16 92.81) (end 137.16 92.71) (width 0.2) (layer F.Cu) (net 7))
 (segment (start 137.86 93.51) (end 137.16 92.81) (width 0.2) (layer F.Cu) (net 7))
 (segment (start 138.385 93.51) (end 137.86 93.51) (width 0.2) (layer F.Cu) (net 7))
 (segment (start 138.65 100.5) (end 138.65 96.05) (width 0.762) (layer F.Cu) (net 7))
 (segment (start 138.385 93.81) (end 138.65 94.075) (width 0.2) (layer F.Cu) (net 7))
 (segment (start 138.385 93.51) (end 138.385 93.81) (width 0.2) (layer F.Cu) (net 7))
 (segment (start 138.65 94.075) (end 138.65 96.05) (width 0.2) (layer F.Cu) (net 7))
 (segment (start 140.734 98.57) (end 142.24 98.57) (width 0.762) (layer F.Cu) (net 7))
 (segment (start 139.954 97.79) (end 140.734 98.57) (width 0.762) (layer F.Cu) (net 7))
 (segment (start 139.954 93.98) (end 139.954 97.79) (width 0.762) (layer F.Cu) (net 7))
 (segment (start 138.385 93.51) (end 139.484 93.51) (width 0.2) (layer F.Cu) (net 7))
 (segment (start 139.484 93.51) (end 139.954 93.98) (width 0.2) (layer F.Cu) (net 7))
 (segment (start 142.24 98.57) (end 143.528 98.57) (width 0.762) (layer F.Cu) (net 7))
 (segment (start 143.773 98.815) (end 146.05 98.815) (width 0.762) (layer F.Cu) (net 7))
 (segment (start 143.528 98.57) (end 143.773 98.815) (width 0.762) (layer F.Cu) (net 7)))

